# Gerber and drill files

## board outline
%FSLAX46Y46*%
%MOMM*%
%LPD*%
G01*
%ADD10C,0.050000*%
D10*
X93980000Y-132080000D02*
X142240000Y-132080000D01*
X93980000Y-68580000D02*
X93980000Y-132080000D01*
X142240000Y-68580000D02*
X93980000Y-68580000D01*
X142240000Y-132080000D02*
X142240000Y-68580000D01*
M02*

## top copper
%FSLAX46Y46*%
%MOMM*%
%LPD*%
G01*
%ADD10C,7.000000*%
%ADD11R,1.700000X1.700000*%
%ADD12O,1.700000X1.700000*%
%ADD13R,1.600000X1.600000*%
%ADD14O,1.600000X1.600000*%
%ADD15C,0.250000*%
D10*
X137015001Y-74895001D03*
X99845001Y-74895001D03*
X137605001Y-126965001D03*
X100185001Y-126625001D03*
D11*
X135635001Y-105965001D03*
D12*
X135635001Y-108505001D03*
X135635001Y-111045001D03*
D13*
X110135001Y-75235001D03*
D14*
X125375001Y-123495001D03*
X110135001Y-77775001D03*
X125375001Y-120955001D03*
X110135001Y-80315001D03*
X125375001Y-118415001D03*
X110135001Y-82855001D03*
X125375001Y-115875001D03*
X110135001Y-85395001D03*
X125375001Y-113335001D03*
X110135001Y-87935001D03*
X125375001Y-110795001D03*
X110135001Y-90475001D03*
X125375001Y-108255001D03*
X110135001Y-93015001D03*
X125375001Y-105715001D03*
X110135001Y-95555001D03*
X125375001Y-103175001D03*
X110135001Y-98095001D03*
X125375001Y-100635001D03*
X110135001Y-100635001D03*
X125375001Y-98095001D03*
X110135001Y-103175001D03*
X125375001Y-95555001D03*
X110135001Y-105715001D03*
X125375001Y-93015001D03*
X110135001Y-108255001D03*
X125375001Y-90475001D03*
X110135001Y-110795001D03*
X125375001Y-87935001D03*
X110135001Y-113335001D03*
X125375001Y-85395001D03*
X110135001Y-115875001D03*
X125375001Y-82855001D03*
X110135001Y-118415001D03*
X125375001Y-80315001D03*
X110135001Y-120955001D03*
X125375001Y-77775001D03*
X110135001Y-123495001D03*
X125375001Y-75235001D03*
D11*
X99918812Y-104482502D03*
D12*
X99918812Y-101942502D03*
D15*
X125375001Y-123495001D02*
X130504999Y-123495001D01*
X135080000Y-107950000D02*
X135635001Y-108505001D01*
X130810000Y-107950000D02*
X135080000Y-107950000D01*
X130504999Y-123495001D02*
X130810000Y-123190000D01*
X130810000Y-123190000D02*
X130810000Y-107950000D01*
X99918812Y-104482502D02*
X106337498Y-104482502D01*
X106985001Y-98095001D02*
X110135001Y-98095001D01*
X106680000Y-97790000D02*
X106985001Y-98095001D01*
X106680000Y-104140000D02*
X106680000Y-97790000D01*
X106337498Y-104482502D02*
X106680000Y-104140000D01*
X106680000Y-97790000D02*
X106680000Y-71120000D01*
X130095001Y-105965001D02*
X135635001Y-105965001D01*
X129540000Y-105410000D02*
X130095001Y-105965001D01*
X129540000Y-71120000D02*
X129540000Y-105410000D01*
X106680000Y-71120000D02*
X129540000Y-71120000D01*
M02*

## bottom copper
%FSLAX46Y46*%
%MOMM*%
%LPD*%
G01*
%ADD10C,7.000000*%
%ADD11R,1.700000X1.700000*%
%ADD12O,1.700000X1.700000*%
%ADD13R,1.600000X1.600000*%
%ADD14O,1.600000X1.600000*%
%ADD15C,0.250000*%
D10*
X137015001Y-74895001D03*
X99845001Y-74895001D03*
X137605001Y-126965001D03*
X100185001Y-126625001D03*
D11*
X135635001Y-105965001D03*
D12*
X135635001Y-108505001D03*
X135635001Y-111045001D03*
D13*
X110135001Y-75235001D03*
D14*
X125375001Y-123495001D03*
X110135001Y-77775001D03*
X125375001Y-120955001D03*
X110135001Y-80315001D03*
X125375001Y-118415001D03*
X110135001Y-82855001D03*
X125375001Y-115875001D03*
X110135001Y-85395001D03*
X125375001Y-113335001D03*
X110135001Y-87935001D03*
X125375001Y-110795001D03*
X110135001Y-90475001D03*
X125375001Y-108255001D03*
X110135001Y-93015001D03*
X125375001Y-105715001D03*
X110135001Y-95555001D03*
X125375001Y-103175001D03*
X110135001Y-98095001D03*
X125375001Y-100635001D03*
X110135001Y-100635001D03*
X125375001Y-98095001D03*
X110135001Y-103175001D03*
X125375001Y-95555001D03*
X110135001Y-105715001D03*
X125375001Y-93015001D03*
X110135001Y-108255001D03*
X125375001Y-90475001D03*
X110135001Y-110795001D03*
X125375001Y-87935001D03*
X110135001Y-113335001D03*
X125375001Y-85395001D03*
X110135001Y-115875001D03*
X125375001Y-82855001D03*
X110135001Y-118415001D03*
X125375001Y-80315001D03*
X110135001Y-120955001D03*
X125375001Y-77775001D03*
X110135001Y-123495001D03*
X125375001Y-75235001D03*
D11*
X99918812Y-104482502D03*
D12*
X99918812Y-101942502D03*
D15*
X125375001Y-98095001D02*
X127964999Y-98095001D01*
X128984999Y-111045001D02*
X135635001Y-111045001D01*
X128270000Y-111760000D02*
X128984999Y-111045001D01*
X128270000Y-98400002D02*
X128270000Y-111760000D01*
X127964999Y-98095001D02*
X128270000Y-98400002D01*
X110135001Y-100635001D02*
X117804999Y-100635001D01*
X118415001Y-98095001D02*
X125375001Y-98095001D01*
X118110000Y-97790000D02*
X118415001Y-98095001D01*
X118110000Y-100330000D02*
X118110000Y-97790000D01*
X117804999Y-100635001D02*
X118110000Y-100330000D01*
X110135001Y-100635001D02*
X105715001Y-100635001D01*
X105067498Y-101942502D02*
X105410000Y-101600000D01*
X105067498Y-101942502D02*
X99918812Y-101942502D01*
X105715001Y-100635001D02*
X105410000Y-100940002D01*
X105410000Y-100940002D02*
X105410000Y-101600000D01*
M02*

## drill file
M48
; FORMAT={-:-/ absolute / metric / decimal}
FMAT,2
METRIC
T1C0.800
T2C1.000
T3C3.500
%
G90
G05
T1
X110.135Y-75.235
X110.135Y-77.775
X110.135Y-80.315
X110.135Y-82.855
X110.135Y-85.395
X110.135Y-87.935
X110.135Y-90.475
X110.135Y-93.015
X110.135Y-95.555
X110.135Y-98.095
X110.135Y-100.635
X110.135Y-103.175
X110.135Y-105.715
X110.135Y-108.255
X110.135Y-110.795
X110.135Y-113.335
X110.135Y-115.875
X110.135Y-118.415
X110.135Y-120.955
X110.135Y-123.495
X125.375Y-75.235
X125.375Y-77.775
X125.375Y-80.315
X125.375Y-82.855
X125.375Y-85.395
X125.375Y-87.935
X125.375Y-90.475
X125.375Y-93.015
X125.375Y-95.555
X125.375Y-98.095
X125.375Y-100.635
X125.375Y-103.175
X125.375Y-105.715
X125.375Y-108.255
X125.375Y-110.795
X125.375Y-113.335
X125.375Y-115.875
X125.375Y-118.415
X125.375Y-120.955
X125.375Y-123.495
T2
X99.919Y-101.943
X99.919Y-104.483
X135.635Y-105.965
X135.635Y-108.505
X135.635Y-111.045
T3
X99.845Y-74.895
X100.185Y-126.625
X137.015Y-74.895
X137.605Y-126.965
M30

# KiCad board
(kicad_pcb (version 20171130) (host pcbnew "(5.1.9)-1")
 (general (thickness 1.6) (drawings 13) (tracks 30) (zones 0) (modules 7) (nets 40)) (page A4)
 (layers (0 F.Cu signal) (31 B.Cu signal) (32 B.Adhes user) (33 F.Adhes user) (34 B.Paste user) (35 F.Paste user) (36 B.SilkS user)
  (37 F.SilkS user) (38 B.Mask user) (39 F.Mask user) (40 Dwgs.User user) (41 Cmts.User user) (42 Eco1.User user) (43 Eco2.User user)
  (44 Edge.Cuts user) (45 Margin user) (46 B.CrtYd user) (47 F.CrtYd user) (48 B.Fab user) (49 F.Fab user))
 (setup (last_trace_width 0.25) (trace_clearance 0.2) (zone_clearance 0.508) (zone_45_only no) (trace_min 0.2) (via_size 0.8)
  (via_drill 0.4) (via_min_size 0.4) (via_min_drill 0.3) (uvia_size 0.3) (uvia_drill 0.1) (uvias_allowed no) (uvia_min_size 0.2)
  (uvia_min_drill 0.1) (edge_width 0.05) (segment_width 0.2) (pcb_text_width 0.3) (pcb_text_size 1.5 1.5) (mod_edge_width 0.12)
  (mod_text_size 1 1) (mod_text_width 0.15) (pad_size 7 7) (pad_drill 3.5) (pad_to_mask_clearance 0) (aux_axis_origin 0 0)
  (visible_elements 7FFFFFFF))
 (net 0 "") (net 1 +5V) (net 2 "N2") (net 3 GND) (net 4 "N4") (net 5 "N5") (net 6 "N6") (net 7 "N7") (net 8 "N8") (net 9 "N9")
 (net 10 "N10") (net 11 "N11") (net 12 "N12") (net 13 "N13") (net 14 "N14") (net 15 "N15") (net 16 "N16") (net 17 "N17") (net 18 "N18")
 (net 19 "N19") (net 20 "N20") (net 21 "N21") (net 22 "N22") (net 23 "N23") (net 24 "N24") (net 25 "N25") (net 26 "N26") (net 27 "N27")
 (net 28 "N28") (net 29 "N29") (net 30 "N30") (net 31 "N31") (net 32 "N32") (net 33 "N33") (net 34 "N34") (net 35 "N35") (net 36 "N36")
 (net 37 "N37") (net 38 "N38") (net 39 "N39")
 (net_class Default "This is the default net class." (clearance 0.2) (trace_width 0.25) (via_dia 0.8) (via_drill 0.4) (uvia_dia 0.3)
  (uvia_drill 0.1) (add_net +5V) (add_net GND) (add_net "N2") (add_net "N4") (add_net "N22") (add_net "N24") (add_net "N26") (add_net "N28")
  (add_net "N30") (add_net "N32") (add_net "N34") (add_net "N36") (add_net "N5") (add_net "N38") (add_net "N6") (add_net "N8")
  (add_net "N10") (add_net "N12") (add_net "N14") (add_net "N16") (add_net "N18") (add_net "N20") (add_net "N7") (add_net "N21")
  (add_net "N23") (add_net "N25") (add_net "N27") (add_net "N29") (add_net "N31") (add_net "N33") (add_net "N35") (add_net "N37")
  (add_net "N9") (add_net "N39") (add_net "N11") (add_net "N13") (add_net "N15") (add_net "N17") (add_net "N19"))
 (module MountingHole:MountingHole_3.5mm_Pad (layer F.Cu) (at 137.015001 74.895001)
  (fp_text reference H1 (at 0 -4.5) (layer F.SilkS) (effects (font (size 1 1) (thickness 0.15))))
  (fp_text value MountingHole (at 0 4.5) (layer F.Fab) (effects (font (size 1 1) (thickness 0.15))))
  (pad 1 thru_hole circle (at 0 0) (size 7 7) (drill 3.5) (layers *.Cu *.Mask)))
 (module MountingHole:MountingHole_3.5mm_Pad (layer F.Cu) (at 99.845001 74.895001)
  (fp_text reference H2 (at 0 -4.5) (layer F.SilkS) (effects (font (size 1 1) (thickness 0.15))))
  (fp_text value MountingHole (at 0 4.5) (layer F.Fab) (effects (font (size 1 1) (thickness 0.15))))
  (pad 1 thru_hole circle (at 0 0) (size 7 7) (drill 3.5) (layers *.Cu *.Mask)))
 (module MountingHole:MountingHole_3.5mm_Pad (layer F.Cu) (at 137.605001 126.965001)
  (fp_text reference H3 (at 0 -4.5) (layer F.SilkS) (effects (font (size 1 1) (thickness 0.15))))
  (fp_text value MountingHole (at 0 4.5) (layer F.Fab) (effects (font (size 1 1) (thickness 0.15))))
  (pad 1 thru_hole circle (at 0 0) (size 7 7) (drill 3.5) (layers *.Cu *.Mask)))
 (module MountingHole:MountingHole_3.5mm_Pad (layer F.Cu) (at 100.185001 126.625001)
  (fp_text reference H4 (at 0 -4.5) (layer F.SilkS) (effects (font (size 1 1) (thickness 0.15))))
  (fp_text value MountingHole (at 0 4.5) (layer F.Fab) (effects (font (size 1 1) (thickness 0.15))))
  (pad 1 thru_hole circle (at 0 0) (size 7 7) (drill 3.5) (layers *.Cu *.Mask)))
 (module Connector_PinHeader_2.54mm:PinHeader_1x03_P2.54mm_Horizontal (layer F.Cu) (at 135.635001 105.965001)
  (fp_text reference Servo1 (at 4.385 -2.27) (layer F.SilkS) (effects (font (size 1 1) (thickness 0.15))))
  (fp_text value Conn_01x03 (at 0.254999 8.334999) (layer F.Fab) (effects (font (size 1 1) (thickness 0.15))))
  (pad 1 thru_hole rect (at 0 0) (size 1.7 1.7) (drill 1) (layers *.Cu *.Mask) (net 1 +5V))
  (pad 2 thru_hole oval (at 0 2.54) (size 1.7 1.7) (drill 1) (layers *.Cu *.Mask) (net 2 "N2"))
  (pad 3 thru_hole oval (at 0 5.08) (size 1.7 1.7) (drill 1) (layers *.Cu *.Mask) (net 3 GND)))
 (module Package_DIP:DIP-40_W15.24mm (layer F.Cu) (at 110.135001 75.235001)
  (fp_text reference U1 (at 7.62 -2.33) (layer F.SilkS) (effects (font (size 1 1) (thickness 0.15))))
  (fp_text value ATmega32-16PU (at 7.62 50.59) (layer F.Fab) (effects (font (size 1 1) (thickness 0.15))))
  (pad 1 thru_hole rect (at 0 0) (size 1.6 1.6) (drill 0.8) (layers *.Cu *.Mask) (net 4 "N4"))
  (pad 21 thru_hole oval (at 15.24 48.26) (size 1.6 1.6) (drill 0.8) (layers *.Cu *.Mask) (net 2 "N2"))
  (pad 2 thru_hole oval (at 0 2.54) (size 1.6 1.6) (drill 0.8) (layers *.Cu *.Mask) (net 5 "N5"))
  (pad 22 thru_hole oval (at 15.24 45.72) (size 1.6 1.6) (drill 0.8) (layers *.Cu *.Mask) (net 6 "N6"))
  (pad 3 thru_hole oval (at 0 5.08) (size 1.6 1.6) (drill 0.8) (layers *.Cu *.Mask) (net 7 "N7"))
  (pad 23 thru_hole oval (at 15.24 43.18) (size 1.6 1.6) (drill 0.8) (layers *.Cu *.Mask) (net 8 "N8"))
  (pad 4 thru_hole oval (at 0 7.62) (size 1.6 1.6) (drill 0.8) (layers *.Cu *.Mask) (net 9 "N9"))
  (pad 24 thru_hole oval (at 15.24 40.64) (size 1.6 1.6) (drill 0.8) (layers *.Cu *.Mask) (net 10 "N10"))
  (pad 5 thru_hole oval (at 0 10.16) (size 1.6 1.6) (drill 0.8) (layers *.Cu *.Mask) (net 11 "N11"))
  (pad 25 thru_hole oval (at 15.24 38.1) (size 1.6 1.6) (drill 0.8) (layers *.Cu *.Mask) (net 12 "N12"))
  (pad 6 thru_hole oval (at 0 12.7) (size 1.6 1.6) (drill 0.8) (layers *.Cu *.Mask) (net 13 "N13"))
  (pad 26 thru_hole oval (at 15.24 35.56) (size 1.6 1.6) (drill 0.8) (layers *.Cu *.Mask) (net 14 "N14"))
  (pad 7 thru_hole oval (at 0 15.24) (size 1.6 1.6) (drill 0.8) (layers *.Cu *.Mask) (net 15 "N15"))
  (pad 27 thru_hole oval (at 15.24 33.02) (size 1.6 1.6) (drill 0.8) (layers *.Cu *.Mask) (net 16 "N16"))
  (pad 8 thru_hole oval (at 0 17.78) (size 1.6 1.6) (drill 0.8) (layers *.Cu *.Mask) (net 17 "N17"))
  (pad 28 thru_hole oval (at 15.24 30.48) (size 1.6 1.6) (drill 0.8) (layers *.Cu *.Mask) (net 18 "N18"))
  (pad 9 thru_hole oval (at 0 20.32) (size 1.6 1.6) (drill 0.8) (layers *.Cu *.Mask) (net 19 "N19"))
  (pad 29 thru_hole oval (at 15.24 27.94) (size 1.6 1.6) (drill 0.8) (layers *.Cu *.Mask) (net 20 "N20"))
  (pad 10 thru_hole oval (at 0 22.86) (size 1.6 1.6) (drill 0.8) (layers *.Cu *.Mask) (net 1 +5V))
  (pad 30 thru_hole oval (at 15.24 25.4) (size 1.6 1.6) (drill 0.8) (layers *.Cu *.Mask) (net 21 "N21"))
  (pad 11 thru_hole oval (at 0 25.4) (size 1.6 1.6) (drill 0.8) (layers *.Cu *.Mask) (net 3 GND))
  (pad 31 thru_hole oval (at 15.24 22.86) (size 1.6 1.6) (drill 0.8) (layers *.Cu *.Mask) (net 3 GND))
  (pad 12 thru_hole oval (at 0 27.94) (size 1.6 1.6) (drill 0.8) (layers *.Cu *.Mask) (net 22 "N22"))
  (pad 32 thru_hole oval (at 15.24 20.32) (size 1.6 1.6) (drill 0.8) (layers *.Cu *.Mask) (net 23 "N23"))
  (pad 13 thru_hole oval (at 0 30.48) (size 1.6 1.6) (drill 0.8) (layers *.Cu *.Mask) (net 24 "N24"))
  (pad 33 thru_hole oval (at 15.24 17.78) (size 1.6 1.6) (drill 0.8) (layers *.Cu *.Mask) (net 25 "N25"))
  (pad 14 thru_hole oval (at 0 33.02) (size 1.6 1.6) (drill 0.8) (layers *.Cu *.Mask) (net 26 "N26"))
  (pad 34 thru_hole oval (at 15.24 15.24) (size 1.6 1.6) (drill 0.8) (layers *.Cu *.Mask) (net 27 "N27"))
  (pad 15 thru_hole oval (at 0 35.56) (size 1.6 1.6) (drill 0.8) (layers *.Cu *.Mask) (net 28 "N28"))
  (pad 35 thru_hole oval (at 15.24 12.7) (size 1.6 1.6) (drill 0.8) (layers *.Cu *.Mask) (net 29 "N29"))
  (pad 16 thru_hole oval (at 0 38.1) (size 1.6 1.6) (drill 0.8) (layers *.Cu *.Mask) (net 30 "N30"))
  (pad 36 thru_hole oval (at 15.24 10.16) (size 1.6 1.6) (drill 0.8) (layers *.Cu *.Mask) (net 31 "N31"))
  (pad 17 thru_hole oval (at 0 40.64) (size 1.6 1.6) (drill 0.8) (layers *.Cu *.Mask) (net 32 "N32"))
  (pad 37 thru_hole oval (at 15.24 7.62) (size 1.6 1.6) (drill 0.8) (layers *.Cu *.Mask) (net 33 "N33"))
  (pad 18 thru_hole oval (at 0 43.18) (size 1.6 1.6) (drill 0.8) (layers *.Cu *.Mask) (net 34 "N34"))
  (pad 38 thru_hole oval (at 15.24 5.08) (size 1.6 1.6) (drill 0.8) (layers *.Cu *.Mask) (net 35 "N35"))
  (pad 19 thru_hole oval (at 0 45.72) (size 1.6 1.6) (drill 0.8) (layers *.Cu *.Mask) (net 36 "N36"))
  (pad 39 thru_hole oval (at 15.24 2.54) (size 1.6 1.6) (drill 0.8) (layers *.Cu *.Mask) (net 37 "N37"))
  (pad 20 thru_hole oval (at 0 48.26) (size 1.6 1.6) (drill 0.8) (layers *.Cu *.Mask) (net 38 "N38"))
  (pad 40 thru_hole oval (at 15.24 0) (size 1.6 1.6) (drill 0.8) (layers *.Cu *.Mask) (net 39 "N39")))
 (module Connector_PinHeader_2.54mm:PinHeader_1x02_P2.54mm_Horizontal (layer F.Cu) (at 99.918812 104.482502 180)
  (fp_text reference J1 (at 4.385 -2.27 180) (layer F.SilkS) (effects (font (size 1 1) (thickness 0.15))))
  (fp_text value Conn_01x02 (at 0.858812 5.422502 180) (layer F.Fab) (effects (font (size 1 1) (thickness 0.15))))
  (pad 1 thru_hole rect (at 0 0 180) (size 1.7 1.7) (drill 1) (layers *.Cu *.Mask) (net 1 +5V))
  (pad 2 thru_hole oval (at 0 2.54 180) (size 1.7 1.7) (drill 1) (layers *.Cu *.Mask) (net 3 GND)))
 (gr_line (start 93.98 132.08) (end 142.24 132.08) (angle 90) (layer Edge.Cuts) (width 0.05))
 (gr_line (start 93.98 68.58) (end 93.98 132.08) (angle 90) (layer Edge.Cuts) (width 0.05))
 (gr_line (start 142.24 68.58) (end 93.98 68.58) (angle 90) (layer Edge.Cuts) (width 0.05))
 (gr_line (start 142.24 132.08) (end 142.24 68.58) (angle 90) (layer Edge.Cuts) (width 0.05))
 (segment (start 125.375001 123.495001) (end 130.504999 123.495001) (width 0.25) (layer F.Cu) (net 2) (status 400000))
 (segment (start 135.08 107.95) (end 135.635001 108.505001) (width 0.25) (layer F.Cu) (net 2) (status C00000))
 (segment (start 130.81 107.95) (end 135.08 107.95) (width 0.25) (layer F.Cu) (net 2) (status 800000))
 (segment (start 130.504999 123.495001) (end 130.81 123.19) (width 0.25) (layer F.Cu) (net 2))
 (segment (start 130.81 123.19) (end 130.81 107.95) (width 0.25) (layer F.Cu) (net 2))
 (segment (start 99.918812 104.482502) (end 106.337498 104.482502) (width 0.25) (layer F.Cu) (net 1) (status 400000))
 (segment (start 106.985001 98.095001) (end 110.135001 98.095001) (width 0.25) (layer F.Cu) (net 1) (status 800000))
 (segment (start 106.68 97.79) (end 106.985001 98.095001) (width 0.25) (layer F.Cu) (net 1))
 (segment (start 106.68 104.14) (end 106.68 97.79) (width 0.25) (layer F.Cu) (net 1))
 (segment (start 106.337498 104.482502) (end 106.68 104.14) (width 0.25) (layer F.Cu) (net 1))
 (segment (start 106.68 97.79) (end 106.68 71.12) (width 0.25) (layer F.Cu) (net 1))
 (segment (start 130.095001 105.965001) (end 135.635001 105.965001) (width 0.25) (layer F.Cu) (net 1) (status 800000))
 (segment (start 129.54 105.41) (end 130.095001 105.965001) (width 0.25) (layer F.Cu) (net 1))
 (segment (start 129.54 71.12) (end 129.54 105.41) (width 0.25) (layer F.Cu) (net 1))
 (segment (start 106.68 71.12) (end 129.54 71.12) (width 0.25) (layer F.Cu) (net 1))
 (segment (start 125.375001 98.095001) (end 127.964999 98.095001) (width 0.25) (layer B.Cu) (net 3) (status 400000))
 (segment (start 128.984999 111.045001) (end 135.635001 111.045001) (width 0.25) (layer B.Cu) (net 3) (status 800000))
 (segment (start 128.27 111.76) (end 128.984999 111.045001) (width 0.25) (layer B.Cu) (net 3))
 (segment (start 128.27 98.400002) (end 128.27 111.76) (width 0.25) (layer B.Cu) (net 3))
 (segment (start 127.964999 98.095001) (end 128.27 98.400002) (width 0.25) (layer B.Cu) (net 3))
 (segment (start 110.135001 100.635001) (end 117.804999 100.635001) (width 0.25) (layer B.Cu) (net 3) (status 400000))
 (segment (start 118.415001 98.095001) (end 125.375001 98.095001) (width 0.25) (layer B.Cu) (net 3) (status 800000))
 (segment (start 118.11 97.79) (end 118.415001 98.095001) (width 0.25) (layer B.Cu) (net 3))
 (segment (start 118.11 100.33) (end 118.11 97.79) (width 0.25) (layer B.Cu) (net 3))
 (segment (start 117.804999 100.635001) (end 118.11 100.33) (width 0.25) (layer B.Cu) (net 3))
 (segment (start 110.135001 100.635001) (end 105.715001 100.635001) (width 0.25) (layer B.Cu) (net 3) (status 400000))
 (segment (start 105.067498 101.942502) (end 105.41 101.6) (width 0.25) (layer B.Cu) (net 3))
 (segment (start 105.067498 101.942502) (end 99.918812 101.942502) (width 0.25) (layer B.Cu) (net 3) (status 800000))
 (segment (start 105.715001 100.635001) (end 105.41 100.940002) (width 0.25) (layer B.Cu) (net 3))
 (segment (start 105.41 100.940002) (end 105.41 101.6) (width 0.25) (layer B.Cu) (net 3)))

